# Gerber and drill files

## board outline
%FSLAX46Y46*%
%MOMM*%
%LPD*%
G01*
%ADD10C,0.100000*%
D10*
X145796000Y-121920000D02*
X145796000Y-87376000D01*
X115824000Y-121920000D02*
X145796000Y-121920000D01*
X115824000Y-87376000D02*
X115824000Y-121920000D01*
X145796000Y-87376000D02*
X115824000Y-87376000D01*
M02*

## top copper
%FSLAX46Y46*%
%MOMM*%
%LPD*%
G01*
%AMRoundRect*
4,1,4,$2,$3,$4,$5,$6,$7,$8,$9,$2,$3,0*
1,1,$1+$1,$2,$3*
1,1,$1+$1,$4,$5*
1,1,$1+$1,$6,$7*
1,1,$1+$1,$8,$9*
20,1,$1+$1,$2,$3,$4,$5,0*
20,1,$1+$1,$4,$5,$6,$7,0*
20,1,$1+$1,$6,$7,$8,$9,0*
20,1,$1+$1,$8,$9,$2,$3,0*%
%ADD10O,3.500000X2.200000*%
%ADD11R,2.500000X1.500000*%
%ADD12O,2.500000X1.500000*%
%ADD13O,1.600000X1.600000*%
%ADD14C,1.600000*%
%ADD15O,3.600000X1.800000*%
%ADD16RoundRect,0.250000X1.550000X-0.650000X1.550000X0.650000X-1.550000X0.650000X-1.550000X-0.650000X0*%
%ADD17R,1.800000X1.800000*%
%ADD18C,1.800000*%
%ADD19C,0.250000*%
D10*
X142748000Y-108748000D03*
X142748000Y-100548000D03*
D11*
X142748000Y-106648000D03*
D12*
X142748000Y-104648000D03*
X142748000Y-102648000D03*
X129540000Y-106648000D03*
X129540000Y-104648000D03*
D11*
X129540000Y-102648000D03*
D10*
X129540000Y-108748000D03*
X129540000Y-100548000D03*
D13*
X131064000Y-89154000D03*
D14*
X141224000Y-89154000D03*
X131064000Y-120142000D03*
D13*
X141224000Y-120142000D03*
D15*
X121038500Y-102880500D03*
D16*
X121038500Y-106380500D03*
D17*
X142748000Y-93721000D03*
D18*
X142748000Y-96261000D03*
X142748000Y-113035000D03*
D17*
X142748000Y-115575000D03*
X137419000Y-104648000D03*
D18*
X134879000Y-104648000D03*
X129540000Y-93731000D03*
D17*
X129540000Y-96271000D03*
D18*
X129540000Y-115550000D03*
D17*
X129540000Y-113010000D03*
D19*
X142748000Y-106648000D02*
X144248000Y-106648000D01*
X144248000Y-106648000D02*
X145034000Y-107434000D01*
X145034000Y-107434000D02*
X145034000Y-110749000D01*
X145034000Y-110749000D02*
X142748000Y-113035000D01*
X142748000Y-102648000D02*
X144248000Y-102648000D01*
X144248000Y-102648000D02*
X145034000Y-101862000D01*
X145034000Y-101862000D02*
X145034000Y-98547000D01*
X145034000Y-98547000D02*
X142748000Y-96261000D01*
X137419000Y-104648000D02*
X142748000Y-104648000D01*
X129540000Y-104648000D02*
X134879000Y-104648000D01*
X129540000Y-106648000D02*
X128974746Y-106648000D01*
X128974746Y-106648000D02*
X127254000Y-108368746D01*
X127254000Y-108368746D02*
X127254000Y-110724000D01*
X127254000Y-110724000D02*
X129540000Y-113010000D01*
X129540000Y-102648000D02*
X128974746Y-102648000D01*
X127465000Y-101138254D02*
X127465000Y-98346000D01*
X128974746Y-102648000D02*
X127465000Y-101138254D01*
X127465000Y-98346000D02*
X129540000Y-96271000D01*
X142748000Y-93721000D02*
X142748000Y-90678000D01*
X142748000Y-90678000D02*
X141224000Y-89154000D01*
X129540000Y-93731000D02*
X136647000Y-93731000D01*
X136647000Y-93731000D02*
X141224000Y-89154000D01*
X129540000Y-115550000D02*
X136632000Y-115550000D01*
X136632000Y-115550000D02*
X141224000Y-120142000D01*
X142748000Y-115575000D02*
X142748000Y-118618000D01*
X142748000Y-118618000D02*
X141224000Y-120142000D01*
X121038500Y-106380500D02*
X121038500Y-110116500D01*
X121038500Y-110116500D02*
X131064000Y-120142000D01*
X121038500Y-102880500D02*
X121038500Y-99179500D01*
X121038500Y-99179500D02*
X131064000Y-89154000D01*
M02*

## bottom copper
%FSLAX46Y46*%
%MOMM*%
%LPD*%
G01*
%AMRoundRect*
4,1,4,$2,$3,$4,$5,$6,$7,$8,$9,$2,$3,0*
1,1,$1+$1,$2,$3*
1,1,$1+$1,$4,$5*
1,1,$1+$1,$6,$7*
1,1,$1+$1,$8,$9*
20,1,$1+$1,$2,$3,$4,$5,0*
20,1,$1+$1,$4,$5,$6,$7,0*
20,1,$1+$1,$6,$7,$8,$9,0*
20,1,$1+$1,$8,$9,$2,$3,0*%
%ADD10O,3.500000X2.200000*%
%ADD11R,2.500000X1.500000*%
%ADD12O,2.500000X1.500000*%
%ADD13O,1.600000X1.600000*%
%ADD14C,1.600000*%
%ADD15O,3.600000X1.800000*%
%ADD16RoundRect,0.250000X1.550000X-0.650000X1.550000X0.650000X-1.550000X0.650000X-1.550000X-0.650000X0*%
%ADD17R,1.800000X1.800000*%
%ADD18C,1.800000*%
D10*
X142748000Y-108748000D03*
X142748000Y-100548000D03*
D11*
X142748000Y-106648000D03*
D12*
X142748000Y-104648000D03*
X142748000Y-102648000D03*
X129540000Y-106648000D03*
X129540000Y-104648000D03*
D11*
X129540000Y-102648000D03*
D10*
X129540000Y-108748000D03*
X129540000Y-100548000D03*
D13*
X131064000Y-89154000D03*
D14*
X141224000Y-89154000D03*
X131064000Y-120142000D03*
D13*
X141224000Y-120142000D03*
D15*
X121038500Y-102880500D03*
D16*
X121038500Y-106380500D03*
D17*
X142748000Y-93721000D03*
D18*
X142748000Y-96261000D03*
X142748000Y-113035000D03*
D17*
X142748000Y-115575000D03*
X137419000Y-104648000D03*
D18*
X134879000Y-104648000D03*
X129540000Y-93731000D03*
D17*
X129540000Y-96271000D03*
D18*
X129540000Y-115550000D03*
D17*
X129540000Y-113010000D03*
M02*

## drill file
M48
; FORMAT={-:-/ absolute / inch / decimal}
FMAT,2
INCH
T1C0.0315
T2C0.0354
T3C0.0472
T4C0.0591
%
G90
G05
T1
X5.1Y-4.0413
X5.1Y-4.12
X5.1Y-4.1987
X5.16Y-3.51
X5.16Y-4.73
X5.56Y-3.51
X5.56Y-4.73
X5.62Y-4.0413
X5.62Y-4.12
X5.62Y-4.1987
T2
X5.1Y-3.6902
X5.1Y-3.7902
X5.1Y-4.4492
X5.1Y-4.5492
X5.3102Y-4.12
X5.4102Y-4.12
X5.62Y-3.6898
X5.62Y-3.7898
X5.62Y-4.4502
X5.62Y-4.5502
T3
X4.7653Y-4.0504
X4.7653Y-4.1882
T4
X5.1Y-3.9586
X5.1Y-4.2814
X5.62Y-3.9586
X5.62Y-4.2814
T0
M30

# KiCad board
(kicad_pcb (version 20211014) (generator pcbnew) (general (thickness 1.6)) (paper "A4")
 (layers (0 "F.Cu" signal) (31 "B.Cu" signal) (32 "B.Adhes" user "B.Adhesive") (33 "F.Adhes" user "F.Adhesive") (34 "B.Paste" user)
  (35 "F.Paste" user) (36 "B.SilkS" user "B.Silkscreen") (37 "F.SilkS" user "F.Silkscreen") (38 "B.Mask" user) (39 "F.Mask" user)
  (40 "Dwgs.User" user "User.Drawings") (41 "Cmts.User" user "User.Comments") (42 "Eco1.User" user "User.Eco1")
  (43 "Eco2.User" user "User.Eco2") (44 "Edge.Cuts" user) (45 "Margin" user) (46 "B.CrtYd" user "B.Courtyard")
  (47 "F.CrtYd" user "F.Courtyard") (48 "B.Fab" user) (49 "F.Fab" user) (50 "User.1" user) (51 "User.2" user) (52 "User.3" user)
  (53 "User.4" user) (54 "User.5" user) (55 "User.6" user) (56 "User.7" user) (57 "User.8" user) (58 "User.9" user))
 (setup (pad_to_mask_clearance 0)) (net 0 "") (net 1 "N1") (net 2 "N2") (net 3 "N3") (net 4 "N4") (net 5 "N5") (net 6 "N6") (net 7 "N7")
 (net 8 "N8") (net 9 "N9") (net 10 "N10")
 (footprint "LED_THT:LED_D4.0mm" (layer "F.Cu") (at 142.748 93.721 -90)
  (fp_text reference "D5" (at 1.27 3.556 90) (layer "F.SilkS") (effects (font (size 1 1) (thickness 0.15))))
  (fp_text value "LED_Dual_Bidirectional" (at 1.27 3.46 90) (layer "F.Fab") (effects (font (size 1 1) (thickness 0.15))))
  (pad "1" thru_hole rect (at 0 0 270) (size 1.8 1.8) (drill 0.9) (layers *.Cu *.Mask) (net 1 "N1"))
  (pad "2" thru_hole circle (at 2.54 0 270) (size 1.8 1.8) (drill 0.9) (layers *.Cu *.Mask) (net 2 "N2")))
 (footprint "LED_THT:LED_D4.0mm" (layer "F.Cu") (at 142.748 115.575 90)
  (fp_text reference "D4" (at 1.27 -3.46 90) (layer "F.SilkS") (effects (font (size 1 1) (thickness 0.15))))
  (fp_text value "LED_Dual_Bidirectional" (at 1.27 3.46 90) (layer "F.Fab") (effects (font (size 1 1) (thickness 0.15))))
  (pad "1" thru_hole rect (at 0 0 90) (size 1.8 1.8) (drill 0.9) (layers *.Cu *.Mask) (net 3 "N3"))
  (pad "2" thru_hole circle (at 2.54 0 90) (size 1.8 1.8) (drill 0.9) (layers *.Cu *.Mask) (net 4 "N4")))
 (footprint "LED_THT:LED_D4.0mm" (layer "F.Cu") (at 137.419 104.648 180)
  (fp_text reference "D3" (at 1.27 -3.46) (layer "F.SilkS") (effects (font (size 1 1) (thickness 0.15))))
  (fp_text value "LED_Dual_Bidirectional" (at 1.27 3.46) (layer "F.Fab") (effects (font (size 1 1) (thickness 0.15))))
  (pad "1" thru_hole rect (at 0 0 180) (size 1.8 1.8) (drill 0.9) (layers *.Cu *.Mask) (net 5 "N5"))
  (pad "2" thru_hole circle (at 2.54 0 180) (size 1.8 1.8) (drill 0.9) (layers *.Cu *.Mask) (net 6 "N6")))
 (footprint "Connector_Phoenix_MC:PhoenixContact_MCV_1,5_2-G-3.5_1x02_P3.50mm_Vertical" (layer "F.Cu") (at 121.0385 106.3805 90)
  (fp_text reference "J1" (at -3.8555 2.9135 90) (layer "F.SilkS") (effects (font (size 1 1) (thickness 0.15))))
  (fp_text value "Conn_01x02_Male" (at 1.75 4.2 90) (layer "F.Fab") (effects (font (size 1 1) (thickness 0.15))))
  (pad "1" thru_hole roundrect (at 0 0 90) (size 1.8 3.6) (drill 1.2) (layers *.Cu *.Mask) (roundrect_rratio 0.1388888889) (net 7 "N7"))
  (pad "2" thru_hole oval (at 3.5 0 90) (size 1.8 3.6) (drill 1.2) (layers *.Cu *.Mask) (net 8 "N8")))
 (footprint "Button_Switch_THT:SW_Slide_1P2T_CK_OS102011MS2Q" (layer "F.Cu") (at 142.748 106.648 90)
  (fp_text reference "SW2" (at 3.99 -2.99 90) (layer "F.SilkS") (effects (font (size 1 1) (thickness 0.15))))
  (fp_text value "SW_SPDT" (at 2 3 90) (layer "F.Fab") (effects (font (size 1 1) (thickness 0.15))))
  (pad "" thru_hole oval (at 6.1 0 90) (size 2.2 3.5) (drill 1.5) (layers *.Cu *.Mask))
  (pad "" thru_hole oval (at -2.1 0 90) (size 2.2 3.5) (drill 1.5) (layers *.Cu *.Mask))
  (pad "1" thru_hole rect (at 0 0 90) (size 1.5 2.5) (drill 0.8) (layers *.Cu *.Mask) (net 4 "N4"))
  (pad "2" thru_hole oval (at 2 0 90) (size 1.5 2.5) (drill 0.8) (layers *.Cu *.Mask) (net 5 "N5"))
  (pad "3" thru_hole oval (at 4 0 90) (size 1.5 2.5) (drill 0.8) (layers *.Cu *.Mask) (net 2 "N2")))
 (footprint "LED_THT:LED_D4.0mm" (layer "F.Cu") (at 129.54 96.271 90)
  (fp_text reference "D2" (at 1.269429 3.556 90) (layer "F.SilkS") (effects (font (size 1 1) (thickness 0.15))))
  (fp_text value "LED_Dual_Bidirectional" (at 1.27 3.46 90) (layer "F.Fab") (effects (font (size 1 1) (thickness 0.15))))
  (pad "1" thru_hole rect (at 0 0 90) (size 1.8 1.8) (drill 0.9) (layers *.Cu *.Mask) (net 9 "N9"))
  (pad "2" thru_hole circle (at 2.54 0 90) (size 1.8 1.8) (drill 0.9) (layers *.Cu *.Mask) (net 1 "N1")))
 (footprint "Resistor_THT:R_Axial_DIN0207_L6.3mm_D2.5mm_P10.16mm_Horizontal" (layer "F.Cu") (at 141.224 89.154 180)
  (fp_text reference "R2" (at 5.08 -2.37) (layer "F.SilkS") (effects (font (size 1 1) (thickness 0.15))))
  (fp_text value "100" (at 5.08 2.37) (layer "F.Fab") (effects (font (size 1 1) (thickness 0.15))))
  (pad "1" thru_hole circle (at 0 0 180) (size 1.6 1.6) (drill 0.8) (layers *.Cu *.Mask) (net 1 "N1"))
  (pad "2" thru_hole oval (at 10.16 0 180) (size 1.6 1.6) (drill 0.8) (layers *.Cu *.Mask) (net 8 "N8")))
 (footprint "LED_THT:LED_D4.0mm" (layer "F.Cu") (at 129.54 113.01 -90)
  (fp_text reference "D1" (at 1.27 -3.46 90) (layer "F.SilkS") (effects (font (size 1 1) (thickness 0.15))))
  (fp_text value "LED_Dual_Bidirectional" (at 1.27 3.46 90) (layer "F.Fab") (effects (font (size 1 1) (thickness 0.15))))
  (pad "1" thru_hole rect (at 0 0 270) (size 1.8 1.8) (drill 0.9) (layers *.Cu *.Mask) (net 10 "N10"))
  (pad "2" thru_hole circle (at 2.54 0 270) (size 1.8 1.8) (drill 0.9) (layers *.Cu *.Mask) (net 3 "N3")))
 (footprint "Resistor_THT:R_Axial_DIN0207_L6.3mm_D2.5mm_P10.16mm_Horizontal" (layer "F.Cu") (at 131.064 120.142)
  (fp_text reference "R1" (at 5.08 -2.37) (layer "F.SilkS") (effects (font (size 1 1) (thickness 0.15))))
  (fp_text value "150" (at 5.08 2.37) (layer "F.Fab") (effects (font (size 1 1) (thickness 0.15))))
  (pad "1" thru_hole circle (at 0 0) (size 1.6 1.6) (drill 0.8) (layers *.Cu *.Mask) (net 7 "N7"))
  (pad "2" thru_hole oval (at 10.16 0) (size 1.6 1.6) (drill 0.8) (layers *.Cu *.Mask) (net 3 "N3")))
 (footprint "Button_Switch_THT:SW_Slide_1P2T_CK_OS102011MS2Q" (layer "F.Cu") (at 129.54 102.648 -90)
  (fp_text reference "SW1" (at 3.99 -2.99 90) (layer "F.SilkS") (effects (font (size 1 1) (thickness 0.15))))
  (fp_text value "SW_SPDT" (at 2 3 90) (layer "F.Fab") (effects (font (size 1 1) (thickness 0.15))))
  (pad "" thru_hole oval (at -2.1 0 270) (size 2.2 3.5) (drill 1.5) (layers *.Cu *.Mask))
  (pad "" thru_hole oval (at 6.1 0 270) (size 2.2 3.5) (drill 1.5) (layers *.Cu *.Mask))
  (pad "1" thru_hole rect (at 0 0 270) (size 1.5 2.5) (drill 0.8) (layers *.Cu *.Mask) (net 9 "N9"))
  (pad "2" thru_hole oval (at 2 0 270) (size 1.5 2.5) (drill 0.8) (layers *.Cu *.Mask) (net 6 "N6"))
  (pad "3" thru_hole oval (at 4 0 270) (size 1.5 2.5) (drill 0.8) (layers *.Cu *.Mask) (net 10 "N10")))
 (gr_line (start 115.824 87.376) (end 115.824 121.92) (layer "Edge.Cuts") (width 0.1))
 (gr_line (start 115.824 121.92) (end 145.796 121.92) (layer "Edge.Cuts") (width 0.1))
 (gr_line (start 145.796 121.92) (end 145.796 87.376) (layer "Edge.Cuts") (width 0.1))
 (gr_line (start 145.796 87.376) (end 115.824 87.376) (layer "Edge.Cuts") (width 0.1))
 (segment (start 127.254 108.368746) (end 127.254 110.724) (width 0.25) (layer "F.Cu") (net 10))
 (segment (start 129.54 106.648) (end 128.974746 106.648) (width 0.25) (layer "F.Cu") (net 10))
 (segment (start 127.254 110.724) (end 129.54 113.01) (width 0.25) (layer "F.Cu") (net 10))
 (segment (start 128.974746 106.648) (end 127.254 108.368746) (width 0.25) (layer "F.Cu") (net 10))
 (segment (start 142.748 118.618) (end 141.224 120.142) (width 0.25) (layer "F.Cu") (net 3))
 (segment (start 136.632 115.55) (end 141.224 120.142) (width 0.25) (layer "F.Cu") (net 3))
 (segment (start 129.54 115.55) (end 136.632 115.55) (width 0.25) (layer "F.Cu") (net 3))
 (segment (start 142.748 115.575) (end 142.748 118.618) (width 0.25) (layer "F.Cu") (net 3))
 (segment (start 128.974746 102.648) (end 127.465 101.138254) (width 0.25) (layer "F.Cu") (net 9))
 (segment (start 129.54 102.648) (end 128.974746 102.648) (width 0.25) (layer "F.Cu") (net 9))
 (segment (start 127.465 98.346) (end 129.54 96.271) (width 0.25) (layer "F.Cu") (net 9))
 (segment (start 127.465 101.138254) (end 127.465 98.346) (width 0.25) (layer "F.Cu") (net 9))
 (segment (start 136.647 93.731) (end 141.224 89.154) (width 0.25) (layer "F.Cu") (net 1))
 (segment (start 142.748 90.678) (end 141.224 89.154) (width 0.25) (layer "F.Cu") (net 1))
 (segment (start 142.748 93.721) (end 142.748 90.678) (width 0.25) (layer "F.Cu") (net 1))
 (segment (start 129.54 93.731) (end 136.647 93.731) (width 0.25) (layer "F.Cu") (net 1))
 (segment (start 137.419 104.648) (end 142.748 104.648) (width 0.25) (layer "F.Cu") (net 5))
 (segment (start 129.54 104.648) (end 134.879 104.648) (width 0.25) (layer "F.Cu") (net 6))
 (segment (start 144.248 106.648) (end 145.034 107.434) (width 0.25) (layer "F.Cu") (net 4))
 (segment (start 142.748 106.648) (end 144.248 106.648) (width 0.25) (layer "F.Cu") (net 4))
 (segment (start 145.034 110.749) (end 142.748 113.035) (width 0.25) (layer "F.Cu") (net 4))
 (segment (start 145.034 107.434) (end 145.034 110.749) (width 0.25) (layer "F.Cu") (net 4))
 (segment (start 145.034 101.862) (end 145.034 98.547) (width 0.25) (layer "F.Cu") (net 2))
 (segment (start 145.034 98.547) (end 142.748 96.261) (width 0.25) (layer "F.Cu") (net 2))
 (segment (start 144.248 102.648) (end 145.034 101.862) (width 0.25) (layer "F.Cu") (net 2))
 (segment (start 142.748 102.648) (end 144.248 102.648) (width 0.25) (layer "F.Cu") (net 2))
 (segment (start 121.0385 110.1165) (end 131.064 120.142) (width 0.25) (layer "F.Cu") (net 7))
 (segment (start 121.0385 106.3805) (end 121.0385 110.1165) (width 0.25) (layer "F.Cu") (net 7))
 (segment (start 121.0385 99.1795) (end 131.064 89.154) (width 0.25) (layer "F.Cu") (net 8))
 (segment (start 121.0385 102.8805) (end 121.0385 99.1795) (width 0.25) (layer "F.Cu") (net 8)))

